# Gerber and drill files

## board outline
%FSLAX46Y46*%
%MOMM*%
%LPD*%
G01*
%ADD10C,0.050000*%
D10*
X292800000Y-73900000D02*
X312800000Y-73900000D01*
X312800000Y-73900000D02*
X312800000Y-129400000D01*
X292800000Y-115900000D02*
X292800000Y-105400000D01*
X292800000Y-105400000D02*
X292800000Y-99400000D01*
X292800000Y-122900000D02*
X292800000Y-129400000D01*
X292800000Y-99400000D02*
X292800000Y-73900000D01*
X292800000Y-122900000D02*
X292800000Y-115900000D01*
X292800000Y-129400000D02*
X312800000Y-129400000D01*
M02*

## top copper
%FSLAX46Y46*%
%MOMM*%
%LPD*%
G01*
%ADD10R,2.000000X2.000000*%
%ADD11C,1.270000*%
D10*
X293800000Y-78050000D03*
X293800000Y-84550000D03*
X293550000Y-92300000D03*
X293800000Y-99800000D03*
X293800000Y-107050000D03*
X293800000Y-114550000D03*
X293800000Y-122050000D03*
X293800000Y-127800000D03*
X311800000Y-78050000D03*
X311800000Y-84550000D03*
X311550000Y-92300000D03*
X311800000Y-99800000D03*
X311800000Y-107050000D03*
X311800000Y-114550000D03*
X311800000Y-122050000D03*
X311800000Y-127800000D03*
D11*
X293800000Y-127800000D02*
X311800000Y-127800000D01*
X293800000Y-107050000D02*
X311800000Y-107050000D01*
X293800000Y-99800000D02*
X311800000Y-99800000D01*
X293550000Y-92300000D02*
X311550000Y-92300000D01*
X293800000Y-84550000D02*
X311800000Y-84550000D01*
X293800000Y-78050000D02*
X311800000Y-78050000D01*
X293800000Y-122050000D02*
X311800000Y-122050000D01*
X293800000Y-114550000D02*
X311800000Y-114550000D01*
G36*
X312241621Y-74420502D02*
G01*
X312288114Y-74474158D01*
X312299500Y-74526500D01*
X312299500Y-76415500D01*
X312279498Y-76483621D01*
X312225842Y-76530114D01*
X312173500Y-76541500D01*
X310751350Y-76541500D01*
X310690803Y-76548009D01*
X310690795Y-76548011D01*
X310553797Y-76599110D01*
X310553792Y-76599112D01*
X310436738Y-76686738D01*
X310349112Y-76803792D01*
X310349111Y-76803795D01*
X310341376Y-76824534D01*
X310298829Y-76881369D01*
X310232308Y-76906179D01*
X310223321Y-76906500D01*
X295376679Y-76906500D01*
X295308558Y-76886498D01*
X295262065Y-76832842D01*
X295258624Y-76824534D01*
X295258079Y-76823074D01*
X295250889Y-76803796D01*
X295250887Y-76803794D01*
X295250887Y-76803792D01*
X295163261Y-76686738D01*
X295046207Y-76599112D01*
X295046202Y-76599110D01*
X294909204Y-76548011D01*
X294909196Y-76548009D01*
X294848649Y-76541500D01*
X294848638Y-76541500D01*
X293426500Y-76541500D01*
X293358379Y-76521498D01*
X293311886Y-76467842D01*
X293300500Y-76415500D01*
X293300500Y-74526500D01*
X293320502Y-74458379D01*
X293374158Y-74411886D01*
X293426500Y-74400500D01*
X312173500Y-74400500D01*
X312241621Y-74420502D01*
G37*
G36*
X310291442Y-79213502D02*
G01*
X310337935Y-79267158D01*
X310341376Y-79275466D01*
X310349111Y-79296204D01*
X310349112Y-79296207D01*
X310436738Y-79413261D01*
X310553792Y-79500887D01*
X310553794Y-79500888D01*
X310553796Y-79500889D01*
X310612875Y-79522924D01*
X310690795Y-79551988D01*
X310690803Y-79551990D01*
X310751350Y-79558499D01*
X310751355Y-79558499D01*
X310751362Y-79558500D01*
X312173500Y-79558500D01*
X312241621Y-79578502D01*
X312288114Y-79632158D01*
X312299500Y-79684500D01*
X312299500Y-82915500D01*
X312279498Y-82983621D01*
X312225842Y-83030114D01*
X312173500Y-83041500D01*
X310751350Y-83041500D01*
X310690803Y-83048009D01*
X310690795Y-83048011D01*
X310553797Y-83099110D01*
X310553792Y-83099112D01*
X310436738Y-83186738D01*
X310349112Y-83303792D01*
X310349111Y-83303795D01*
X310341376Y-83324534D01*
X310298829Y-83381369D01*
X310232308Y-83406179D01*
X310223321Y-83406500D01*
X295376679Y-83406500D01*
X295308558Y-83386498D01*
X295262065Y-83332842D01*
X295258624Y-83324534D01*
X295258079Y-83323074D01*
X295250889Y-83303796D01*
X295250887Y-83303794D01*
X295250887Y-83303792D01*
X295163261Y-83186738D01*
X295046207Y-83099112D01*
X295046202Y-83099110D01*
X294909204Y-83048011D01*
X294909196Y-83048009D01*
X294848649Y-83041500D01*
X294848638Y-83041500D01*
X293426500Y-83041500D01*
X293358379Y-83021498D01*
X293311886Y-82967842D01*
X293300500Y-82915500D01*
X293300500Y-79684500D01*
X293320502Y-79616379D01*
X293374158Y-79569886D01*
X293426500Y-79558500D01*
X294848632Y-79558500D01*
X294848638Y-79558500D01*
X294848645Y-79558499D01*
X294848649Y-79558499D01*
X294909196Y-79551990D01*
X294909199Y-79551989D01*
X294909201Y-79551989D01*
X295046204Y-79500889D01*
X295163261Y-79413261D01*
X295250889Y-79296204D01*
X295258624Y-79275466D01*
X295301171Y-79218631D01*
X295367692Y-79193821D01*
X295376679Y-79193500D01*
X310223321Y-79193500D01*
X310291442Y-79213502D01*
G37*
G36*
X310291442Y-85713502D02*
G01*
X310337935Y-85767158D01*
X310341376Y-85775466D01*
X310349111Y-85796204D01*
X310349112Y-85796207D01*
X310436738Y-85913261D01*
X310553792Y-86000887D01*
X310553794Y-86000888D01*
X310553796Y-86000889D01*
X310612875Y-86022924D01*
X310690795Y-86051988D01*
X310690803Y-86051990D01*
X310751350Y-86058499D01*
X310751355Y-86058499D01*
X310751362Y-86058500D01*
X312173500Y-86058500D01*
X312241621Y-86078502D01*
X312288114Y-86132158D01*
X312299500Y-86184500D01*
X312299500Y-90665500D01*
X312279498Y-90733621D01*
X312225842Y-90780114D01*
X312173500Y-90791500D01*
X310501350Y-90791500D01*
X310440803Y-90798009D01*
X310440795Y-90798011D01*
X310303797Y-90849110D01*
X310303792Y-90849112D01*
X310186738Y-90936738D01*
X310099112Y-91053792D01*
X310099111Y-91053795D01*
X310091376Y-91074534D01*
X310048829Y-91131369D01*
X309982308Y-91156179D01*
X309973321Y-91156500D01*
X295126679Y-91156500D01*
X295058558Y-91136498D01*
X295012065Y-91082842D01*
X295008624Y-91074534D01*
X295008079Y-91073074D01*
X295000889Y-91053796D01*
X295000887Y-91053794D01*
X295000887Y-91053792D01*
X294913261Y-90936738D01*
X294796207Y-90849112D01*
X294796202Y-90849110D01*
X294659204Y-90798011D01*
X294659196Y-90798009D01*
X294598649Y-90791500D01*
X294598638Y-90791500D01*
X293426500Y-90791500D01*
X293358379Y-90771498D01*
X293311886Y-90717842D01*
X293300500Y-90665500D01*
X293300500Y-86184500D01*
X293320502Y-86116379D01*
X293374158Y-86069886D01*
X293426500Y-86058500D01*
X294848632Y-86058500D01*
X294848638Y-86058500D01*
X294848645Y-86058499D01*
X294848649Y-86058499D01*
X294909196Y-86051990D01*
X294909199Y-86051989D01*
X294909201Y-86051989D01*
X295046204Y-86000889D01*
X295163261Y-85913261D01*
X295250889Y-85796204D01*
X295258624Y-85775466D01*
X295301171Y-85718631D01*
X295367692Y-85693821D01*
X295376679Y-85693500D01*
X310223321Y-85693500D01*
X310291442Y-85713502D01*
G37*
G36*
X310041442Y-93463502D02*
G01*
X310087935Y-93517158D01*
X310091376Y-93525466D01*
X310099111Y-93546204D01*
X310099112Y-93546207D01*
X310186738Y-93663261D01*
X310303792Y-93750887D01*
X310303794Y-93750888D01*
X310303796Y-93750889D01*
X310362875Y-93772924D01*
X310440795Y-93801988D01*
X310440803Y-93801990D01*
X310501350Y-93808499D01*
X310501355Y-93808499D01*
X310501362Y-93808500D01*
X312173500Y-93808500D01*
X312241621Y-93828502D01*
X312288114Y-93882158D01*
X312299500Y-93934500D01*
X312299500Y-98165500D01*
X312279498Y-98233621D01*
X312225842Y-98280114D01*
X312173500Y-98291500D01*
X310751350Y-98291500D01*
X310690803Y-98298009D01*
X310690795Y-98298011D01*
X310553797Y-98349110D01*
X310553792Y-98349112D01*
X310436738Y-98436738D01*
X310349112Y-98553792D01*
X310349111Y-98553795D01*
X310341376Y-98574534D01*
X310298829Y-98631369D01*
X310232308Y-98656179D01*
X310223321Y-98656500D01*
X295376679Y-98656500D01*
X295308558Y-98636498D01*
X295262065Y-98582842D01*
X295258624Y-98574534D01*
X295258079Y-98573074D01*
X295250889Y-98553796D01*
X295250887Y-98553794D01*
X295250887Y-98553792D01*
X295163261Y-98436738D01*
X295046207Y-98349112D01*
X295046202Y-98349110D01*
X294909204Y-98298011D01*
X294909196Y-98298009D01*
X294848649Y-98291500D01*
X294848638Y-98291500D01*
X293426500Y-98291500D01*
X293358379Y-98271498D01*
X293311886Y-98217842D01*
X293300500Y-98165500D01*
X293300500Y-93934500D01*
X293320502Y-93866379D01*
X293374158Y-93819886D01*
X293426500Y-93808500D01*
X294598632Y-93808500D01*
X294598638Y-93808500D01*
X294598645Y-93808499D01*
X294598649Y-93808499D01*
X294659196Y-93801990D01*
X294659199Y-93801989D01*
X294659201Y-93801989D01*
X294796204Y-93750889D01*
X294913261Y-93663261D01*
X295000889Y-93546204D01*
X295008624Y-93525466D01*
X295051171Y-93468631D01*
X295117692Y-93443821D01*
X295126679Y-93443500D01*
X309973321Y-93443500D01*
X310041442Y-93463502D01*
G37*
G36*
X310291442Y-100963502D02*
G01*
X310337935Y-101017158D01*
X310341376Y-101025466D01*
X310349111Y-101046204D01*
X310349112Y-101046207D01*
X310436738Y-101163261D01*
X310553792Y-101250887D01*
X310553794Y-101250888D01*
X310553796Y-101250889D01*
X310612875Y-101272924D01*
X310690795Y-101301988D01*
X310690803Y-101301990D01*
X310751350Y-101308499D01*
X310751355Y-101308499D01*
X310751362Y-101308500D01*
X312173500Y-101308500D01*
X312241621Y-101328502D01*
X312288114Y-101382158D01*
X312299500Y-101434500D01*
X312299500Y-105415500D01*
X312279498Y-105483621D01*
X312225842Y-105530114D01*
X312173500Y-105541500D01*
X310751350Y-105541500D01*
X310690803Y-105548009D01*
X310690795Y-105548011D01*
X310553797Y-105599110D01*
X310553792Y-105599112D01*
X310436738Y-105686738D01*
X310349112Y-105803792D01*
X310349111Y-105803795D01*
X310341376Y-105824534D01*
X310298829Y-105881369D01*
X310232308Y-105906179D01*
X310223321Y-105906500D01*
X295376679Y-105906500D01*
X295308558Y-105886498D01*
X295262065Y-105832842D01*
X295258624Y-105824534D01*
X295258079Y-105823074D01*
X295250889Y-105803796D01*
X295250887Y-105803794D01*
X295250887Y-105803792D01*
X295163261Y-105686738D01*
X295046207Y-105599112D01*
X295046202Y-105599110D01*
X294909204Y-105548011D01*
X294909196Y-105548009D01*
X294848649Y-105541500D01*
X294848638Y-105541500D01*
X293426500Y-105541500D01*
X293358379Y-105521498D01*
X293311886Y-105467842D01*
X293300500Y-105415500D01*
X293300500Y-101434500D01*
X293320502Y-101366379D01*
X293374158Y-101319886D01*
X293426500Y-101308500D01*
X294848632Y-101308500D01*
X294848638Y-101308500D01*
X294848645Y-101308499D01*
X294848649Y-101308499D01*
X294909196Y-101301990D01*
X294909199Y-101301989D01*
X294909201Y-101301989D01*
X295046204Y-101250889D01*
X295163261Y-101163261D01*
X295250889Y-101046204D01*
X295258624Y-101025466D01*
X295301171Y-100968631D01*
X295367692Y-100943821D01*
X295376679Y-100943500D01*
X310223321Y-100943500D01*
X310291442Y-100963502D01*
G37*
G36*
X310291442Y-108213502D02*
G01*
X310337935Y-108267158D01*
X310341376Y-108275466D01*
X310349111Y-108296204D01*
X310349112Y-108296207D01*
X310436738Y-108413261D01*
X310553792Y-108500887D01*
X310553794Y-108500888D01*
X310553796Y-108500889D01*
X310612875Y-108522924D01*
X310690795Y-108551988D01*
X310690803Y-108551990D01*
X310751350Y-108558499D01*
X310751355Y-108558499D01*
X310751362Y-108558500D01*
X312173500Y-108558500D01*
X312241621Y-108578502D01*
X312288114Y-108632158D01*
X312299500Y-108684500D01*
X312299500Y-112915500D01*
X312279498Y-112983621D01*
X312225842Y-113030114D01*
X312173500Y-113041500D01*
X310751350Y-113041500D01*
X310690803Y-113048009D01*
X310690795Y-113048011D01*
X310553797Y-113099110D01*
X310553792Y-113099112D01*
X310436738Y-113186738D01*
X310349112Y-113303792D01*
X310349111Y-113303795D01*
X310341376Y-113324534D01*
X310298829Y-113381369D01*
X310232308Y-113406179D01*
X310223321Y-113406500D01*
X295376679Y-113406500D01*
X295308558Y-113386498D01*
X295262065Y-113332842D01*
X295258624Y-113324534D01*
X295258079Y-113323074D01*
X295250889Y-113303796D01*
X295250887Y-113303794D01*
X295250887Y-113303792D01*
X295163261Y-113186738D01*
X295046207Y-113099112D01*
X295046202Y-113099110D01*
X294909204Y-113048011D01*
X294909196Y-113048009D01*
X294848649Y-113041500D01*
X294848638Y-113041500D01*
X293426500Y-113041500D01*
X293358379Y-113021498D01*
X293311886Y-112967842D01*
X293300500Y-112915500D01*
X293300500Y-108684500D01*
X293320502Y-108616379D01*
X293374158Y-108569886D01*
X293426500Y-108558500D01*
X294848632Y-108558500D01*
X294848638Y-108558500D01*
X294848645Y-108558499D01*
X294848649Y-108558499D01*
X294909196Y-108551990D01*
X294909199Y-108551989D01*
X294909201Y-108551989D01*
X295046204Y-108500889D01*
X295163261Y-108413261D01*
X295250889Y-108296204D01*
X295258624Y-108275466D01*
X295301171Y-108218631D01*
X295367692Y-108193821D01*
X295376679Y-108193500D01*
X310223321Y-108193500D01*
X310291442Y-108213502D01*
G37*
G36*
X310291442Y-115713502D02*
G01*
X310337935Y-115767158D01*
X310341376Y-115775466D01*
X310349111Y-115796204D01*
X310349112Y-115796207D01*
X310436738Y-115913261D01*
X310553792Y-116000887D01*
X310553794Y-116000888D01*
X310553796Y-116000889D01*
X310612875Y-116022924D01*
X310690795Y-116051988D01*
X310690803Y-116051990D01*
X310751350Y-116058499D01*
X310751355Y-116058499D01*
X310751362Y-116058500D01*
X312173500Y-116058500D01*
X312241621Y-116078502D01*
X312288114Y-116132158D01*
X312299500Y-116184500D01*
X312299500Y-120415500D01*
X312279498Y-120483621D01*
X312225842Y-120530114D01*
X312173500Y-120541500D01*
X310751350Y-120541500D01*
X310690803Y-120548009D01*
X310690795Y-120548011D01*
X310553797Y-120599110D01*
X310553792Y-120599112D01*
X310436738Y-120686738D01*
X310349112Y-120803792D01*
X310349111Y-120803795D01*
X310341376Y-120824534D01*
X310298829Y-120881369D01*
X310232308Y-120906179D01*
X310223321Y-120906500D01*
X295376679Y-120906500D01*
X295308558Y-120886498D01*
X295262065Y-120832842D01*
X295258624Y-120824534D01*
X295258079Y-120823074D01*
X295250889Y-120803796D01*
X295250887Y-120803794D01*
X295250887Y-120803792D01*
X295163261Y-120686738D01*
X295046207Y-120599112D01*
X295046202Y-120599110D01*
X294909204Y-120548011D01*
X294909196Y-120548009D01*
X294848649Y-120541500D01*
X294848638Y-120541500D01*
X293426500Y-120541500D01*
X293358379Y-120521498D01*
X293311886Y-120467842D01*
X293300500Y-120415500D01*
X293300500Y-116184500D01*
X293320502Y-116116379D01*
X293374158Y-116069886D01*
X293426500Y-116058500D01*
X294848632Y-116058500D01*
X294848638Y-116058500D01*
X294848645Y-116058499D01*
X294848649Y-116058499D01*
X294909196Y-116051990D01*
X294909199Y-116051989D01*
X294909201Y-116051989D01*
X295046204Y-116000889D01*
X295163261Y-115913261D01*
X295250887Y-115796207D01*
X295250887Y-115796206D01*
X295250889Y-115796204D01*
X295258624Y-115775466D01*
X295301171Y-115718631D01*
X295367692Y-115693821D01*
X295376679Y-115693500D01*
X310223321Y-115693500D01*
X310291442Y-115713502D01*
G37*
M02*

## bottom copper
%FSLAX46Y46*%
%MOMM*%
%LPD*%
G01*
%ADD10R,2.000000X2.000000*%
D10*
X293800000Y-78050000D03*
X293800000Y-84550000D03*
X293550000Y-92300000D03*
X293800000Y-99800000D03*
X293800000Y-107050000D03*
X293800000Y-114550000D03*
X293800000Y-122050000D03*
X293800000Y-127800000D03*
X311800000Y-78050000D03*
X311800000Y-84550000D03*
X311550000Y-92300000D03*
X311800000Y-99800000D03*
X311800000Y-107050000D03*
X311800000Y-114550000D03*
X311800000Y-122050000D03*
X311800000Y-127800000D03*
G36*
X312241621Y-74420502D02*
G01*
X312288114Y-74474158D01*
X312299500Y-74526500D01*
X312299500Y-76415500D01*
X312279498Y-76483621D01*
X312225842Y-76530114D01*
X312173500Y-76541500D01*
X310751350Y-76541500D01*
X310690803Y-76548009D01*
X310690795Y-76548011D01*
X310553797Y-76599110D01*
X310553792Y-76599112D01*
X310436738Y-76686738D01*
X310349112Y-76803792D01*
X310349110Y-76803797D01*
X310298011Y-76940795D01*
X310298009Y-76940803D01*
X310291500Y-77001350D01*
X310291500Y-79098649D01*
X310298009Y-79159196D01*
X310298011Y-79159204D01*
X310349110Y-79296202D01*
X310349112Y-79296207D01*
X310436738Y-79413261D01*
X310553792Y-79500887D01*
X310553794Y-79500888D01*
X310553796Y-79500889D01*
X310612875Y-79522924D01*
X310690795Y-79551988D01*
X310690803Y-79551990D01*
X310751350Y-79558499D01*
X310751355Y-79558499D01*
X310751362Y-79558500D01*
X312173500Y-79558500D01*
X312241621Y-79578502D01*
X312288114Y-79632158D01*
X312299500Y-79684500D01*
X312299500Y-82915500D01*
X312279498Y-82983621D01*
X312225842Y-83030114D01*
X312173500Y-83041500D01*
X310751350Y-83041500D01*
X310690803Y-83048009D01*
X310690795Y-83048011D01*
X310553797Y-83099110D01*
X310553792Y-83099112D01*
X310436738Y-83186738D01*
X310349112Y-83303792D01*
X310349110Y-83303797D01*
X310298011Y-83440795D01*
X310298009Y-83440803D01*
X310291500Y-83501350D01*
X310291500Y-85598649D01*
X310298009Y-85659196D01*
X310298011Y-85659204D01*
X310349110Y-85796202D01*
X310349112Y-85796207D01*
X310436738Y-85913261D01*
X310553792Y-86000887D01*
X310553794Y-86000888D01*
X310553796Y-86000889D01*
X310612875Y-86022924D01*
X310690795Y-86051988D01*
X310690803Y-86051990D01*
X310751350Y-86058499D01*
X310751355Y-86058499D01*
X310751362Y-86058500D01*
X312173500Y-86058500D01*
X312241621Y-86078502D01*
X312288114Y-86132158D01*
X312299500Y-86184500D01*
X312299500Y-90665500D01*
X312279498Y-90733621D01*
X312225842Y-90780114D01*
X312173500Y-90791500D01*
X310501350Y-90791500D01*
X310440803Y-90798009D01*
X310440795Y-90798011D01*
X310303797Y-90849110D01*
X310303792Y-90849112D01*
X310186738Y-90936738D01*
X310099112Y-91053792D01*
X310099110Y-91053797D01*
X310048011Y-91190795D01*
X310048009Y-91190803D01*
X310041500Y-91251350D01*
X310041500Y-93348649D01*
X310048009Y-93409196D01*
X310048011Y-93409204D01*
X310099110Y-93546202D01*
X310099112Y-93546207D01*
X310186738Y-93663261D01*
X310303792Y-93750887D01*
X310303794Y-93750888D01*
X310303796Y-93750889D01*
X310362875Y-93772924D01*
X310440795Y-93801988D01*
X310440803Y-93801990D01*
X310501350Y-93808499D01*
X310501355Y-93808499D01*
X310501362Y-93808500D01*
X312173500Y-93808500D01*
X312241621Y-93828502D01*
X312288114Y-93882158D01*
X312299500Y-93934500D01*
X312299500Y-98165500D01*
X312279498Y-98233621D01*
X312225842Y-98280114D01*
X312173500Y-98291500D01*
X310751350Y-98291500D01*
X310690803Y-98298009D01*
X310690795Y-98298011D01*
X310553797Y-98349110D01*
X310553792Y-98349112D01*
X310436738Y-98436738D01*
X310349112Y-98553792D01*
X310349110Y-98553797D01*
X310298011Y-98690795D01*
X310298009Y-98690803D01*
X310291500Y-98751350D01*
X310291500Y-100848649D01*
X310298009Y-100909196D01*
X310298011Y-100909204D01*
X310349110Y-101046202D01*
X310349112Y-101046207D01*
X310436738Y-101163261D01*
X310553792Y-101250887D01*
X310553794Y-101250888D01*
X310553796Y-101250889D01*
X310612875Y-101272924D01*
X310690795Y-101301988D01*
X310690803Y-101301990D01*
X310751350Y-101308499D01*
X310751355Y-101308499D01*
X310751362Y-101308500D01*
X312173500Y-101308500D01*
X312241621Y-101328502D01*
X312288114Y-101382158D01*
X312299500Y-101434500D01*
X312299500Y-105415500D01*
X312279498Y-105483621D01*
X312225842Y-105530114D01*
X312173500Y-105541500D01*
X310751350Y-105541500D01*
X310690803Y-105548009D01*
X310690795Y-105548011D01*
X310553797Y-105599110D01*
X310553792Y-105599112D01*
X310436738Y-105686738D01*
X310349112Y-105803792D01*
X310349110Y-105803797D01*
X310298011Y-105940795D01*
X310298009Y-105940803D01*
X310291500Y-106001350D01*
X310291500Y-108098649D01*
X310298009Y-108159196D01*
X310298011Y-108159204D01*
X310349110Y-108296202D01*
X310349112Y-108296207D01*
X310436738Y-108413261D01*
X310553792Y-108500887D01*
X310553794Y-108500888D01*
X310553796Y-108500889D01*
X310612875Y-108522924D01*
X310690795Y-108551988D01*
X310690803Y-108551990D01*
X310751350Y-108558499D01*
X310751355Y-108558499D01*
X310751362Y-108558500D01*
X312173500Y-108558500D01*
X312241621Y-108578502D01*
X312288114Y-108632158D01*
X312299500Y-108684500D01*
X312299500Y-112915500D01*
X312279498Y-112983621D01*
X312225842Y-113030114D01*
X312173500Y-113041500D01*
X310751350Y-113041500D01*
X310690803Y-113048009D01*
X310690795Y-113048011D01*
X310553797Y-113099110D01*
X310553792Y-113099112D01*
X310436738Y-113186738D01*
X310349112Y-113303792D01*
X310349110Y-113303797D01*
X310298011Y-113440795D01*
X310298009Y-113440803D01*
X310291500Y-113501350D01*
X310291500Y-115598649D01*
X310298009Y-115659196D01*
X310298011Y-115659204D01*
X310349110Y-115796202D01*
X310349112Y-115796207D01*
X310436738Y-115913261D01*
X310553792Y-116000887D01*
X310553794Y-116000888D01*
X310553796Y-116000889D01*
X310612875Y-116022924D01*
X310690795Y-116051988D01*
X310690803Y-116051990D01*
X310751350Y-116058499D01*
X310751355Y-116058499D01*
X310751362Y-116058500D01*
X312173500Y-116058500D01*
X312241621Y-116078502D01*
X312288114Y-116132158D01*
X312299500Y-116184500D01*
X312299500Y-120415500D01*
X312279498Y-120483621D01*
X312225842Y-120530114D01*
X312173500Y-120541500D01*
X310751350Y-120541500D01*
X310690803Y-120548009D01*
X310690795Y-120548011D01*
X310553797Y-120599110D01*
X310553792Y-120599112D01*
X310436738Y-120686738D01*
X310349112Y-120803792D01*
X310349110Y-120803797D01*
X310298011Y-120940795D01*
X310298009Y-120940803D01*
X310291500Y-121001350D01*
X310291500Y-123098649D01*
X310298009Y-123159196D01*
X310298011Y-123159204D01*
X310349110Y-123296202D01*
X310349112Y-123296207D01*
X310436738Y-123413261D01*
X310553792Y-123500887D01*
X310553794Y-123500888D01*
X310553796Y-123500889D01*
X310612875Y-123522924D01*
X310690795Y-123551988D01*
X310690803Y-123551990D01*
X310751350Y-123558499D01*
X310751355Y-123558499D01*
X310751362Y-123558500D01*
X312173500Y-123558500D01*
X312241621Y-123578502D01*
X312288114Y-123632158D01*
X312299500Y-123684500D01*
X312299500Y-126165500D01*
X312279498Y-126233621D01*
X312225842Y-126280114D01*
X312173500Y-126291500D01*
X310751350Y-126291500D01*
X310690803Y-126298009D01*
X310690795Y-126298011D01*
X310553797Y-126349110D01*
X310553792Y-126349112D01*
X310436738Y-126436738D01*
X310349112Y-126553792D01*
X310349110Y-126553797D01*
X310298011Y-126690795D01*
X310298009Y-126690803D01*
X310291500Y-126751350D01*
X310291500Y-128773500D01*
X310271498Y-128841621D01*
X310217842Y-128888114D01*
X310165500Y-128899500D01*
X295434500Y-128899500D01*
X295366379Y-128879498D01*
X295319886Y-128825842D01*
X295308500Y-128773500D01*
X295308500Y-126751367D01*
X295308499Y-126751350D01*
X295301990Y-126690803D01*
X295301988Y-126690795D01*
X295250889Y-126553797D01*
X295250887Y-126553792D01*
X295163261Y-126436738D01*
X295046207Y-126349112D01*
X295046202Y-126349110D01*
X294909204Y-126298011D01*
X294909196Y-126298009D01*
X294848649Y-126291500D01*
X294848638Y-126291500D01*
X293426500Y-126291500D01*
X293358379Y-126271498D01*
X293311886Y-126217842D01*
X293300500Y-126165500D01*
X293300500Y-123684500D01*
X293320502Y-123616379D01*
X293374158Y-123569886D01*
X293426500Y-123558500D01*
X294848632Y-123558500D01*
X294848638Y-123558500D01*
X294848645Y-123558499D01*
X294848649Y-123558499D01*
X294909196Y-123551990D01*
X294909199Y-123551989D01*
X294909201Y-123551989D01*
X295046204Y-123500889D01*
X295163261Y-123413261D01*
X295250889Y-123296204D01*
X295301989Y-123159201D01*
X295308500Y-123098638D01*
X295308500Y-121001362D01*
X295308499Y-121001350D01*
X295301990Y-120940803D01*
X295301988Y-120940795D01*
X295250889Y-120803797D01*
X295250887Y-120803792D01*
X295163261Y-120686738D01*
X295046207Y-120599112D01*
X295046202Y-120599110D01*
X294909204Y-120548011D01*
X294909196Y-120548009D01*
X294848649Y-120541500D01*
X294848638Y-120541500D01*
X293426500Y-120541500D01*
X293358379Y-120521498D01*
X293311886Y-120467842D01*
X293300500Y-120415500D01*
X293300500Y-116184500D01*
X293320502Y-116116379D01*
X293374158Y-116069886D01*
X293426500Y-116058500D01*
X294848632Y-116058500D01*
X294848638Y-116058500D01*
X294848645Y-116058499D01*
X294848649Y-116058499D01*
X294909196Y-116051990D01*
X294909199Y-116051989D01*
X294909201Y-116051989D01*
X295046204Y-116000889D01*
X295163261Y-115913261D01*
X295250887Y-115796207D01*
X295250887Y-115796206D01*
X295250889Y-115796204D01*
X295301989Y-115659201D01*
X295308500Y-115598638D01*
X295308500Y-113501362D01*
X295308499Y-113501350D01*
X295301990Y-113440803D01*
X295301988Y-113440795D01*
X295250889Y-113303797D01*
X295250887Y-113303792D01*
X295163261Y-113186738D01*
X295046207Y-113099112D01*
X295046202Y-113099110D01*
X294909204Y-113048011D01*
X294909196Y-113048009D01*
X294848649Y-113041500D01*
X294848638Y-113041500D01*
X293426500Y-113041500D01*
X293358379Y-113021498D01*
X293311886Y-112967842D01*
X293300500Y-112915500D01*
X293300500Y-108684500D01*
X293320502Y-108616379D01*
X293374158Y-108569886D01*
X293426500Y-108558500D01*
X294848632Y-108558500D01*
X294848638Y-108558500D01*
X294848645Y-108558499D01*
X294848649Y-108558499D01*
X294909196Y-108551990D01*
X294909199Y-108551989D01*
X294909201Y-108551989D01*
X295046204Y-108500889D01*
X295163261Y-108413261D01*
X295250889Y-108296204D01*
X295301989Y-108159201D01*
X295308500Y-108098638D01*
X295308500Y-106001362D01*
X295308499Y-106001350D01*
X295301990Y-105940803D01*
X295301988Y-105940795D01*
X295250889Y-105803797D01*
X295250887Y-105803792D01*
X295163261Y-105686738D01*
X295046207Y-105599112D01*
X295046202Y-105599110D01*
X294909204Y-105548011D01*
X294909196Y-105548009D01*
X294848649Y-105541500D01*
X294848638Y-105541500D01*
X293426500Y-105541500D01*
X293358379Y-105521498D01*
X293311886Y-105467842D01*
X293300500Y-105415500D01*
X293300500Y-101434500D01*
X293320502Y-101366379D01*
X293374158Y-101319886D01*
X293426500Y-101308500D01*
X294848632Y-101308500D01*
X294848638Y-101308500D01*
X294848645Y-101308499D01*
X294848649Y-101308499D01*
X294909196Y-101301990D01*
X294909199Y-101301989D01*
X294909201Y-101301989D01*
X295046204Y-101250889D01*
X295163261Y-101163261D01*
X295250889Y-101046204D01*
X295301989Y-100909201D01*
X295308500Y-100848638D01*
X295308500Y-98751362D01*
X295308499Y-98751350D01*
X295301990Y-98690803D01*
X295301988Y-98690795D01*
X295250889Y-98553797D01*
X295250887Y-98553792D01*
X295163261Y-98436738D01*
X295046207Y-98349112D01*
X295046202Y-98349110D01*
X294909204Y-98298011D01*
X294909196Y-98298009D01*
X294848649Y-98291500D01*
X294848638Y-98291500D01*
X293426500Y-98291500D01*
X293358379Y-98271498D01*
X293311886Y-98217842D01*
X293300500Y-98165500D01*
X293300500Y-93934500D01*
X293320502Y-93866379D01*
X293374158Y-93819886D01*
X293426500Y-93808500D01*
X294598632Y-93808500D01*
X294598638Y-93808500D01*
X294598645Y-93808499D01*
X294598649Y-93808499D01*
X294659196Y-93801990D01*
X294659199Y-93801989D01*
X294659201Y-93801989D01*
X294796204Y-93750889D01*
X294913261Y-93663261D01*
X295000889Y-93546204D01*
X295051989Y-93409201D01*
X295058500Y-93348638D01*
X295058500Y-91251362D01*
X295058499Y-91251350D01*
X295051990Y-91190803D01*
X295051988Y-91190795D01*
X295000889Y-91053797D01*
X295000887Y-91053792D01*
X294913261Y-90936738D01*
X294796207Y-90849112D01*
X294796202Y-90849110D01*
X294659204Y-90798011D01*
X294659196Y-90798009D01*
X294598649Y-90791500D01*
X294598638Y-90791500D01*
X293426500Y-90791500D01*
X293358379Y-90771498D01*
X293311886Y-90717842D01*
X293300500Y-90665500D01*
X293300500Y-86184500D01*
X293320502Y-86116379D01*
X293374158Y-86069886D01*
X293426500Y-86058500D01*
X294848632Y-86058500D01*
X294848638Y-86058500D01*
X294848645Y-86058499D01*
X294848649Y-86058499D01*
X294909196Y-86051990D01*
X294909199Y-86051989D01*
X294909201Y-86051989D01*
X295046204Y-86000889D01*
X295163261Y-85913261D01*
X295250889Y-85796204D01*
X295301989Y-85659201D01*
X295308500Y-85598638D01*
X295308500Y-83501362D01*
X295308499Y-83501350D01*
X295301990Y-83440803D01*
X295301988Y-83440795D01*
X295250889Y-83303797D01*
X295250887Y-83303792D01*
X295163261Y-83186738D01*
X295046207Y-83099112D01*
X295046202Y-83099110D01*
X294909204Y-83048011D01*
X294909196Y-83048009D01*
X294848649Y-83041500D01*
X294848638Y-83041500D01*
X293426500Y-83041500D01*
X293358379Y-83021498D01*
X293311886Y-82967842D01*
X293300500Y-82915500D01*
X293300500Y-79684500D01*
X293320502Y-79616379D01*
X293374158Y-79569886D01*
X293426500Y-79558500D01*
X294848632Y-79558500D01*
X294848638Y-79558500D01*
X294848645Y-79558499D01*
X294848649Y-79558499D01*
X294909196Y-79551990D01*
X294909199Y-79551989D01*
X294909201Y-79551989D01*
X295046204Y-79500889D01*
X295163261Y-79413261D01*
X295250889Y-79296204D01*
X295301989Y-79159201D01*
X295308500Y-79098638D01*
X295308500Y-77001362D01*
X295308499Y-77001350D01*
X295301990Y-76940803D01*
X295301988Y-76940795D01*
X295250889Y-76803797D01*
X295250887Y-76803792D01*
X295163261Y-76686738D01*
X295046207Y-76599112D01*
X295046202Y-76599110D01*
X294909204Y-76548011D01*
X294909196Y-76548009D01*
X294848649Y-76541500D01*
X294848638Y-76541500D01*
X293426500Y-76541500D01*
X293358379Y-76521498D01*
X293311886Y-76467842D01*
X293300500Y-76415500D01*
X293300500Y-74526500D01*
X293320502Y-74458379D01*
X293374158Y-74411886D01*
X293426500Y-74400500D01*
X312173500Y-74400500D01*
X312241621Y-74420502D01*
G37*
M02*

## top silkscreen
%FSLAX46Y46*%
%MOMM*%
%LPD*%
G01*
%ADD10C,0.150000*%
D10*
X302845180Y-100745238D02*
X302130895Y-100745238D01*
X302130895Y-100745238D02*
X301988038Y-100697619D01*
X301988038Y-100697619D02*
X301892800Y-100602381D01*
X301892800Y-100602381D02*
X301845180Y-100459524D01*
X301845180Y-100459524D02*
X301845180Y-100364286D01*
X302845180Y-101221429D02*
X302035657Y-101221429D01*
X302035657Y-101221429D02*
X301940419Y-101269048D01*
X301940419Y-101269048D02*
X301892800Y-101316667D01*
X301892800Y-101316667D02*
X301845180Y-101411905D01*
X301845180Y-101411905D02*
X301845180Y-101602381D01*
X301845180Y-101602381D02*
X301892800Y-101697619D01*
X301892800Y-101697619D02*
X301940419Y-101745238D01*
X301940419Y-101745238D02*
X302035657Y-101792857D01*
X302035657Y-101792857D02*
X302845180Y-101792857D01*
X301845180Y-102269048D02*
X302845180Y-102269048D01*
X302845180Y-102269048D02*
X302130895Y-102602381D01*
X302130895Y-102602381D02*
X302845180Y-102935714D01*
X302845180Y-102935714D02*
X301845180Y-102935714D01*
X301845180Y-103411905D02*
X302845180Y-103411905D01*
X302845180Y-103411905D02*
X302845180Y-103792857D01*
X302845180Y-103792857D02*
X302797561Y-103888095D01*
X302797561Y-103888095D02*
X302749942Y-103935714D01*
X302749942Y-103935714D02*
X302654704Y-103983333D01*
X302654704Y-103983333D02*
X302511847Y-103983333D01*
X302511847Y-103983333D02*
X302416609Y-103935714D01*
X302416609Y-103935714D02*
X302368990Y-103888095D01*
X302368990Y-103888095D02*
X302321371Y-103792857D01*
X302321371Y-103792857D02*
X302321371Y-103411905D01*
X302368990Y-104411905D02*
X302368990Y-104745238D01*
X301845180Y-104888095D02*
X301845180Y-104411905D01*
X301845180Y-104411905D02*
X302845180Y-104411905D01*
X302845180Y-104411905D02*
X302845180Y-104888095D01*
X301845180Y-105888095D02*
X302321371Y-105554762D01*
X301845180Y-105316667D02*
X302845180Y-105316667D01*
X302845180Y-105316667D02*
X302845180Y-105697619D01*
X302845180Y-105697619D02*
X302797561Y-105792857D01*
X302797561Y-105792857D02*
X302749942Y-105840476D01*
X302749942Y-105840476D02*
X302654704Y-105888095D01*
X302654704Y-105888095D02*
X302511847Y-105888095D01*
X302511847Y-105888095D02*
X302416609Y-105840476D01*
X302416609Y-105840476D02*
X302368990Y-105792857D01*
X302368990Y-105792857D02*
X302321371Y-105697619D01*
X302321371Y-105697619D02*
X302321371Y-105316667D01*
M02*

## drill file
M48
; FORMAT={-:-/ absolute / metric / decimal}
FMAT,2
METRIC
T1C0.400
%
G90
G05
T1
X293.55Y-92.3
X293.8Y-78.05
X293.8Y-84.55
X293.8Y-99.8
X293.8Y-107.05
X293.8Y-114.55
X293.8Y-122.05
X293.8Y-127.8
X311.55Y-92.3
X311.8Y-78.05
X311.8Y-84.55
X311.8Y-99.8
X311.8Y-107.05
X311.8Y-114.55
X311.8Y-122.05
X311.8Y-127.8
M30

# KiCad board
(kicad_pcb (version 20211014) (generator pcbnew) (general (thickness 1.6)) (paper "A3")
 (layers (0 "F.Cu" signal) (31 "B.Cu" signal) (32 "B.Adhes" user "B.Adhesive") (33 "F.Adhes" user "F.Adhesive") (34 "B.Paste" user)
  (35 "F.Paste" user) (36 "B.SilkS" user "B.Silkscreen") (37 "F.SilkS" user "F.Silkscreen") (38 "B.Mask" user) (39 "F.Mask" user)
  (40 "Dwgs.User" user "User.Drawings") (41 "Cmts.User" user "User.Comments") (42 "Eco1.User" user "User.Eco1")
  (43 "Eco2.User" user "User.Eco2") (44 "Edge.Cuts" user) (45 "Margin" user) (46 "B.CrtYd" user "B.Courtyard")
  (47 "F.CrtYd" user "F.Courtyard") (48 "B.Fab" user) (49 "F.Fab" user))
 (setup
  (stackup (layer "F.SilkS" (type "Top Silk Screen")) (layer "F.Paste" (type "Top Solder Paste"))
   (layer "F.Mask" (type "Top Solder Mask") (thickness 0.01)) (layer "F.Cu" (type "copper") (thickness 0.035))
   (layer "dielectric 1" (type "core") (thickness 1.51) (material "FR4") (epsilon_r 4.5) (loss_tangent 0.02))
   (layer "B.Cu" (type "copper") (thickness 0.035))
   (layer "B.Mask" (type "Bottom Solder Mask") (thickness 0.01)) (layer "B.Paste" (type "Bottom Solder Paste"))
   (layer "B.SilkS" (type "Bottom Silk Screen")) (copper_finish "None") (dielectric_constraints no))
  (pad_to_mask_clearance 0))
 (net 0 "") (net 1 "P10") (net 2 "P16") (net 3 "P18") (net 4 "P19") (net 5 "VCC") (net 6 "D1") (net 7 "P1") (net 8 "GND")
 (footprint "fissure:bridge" (layer "F.Cu") (at 293.8 107.55 90)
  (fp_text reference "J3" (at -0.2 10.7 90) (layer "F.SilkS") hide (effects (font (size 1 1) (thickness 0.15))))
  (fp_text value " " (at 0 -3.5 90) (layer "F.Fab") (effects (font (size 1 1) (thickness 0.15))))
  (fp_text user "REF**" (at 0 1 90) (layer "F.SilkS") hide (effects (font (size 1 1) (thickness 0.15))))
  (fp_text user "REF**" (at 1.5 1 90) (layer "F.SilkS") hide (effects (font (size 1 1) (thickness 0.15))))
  (pad "1" thru_hole rect (at 29.5 0 90) (size 2 2) (drill 0.4) (layers *.Cu *.Mask) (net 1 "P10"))
  (pad "2" thru_hole rect (at 23 0 90) (size 2 2) (drill 0.4) (layers F&B.Cu *.Mask) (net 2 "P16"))
  (pad "3" thru_hole rect (at 15.25 -0.25 90) (size 2 2) (drill 0.4) (layers F&B.Cu *.Mask) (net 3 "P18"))
  (pad "4" thru_hole rect (at 7.75 0 90) (size 2 2) (drill 0.4) (layers F&B.Cu *.Mask) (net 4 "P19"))
  (pad "5" thru_hole rect (at 0.5 0 90) (size 2 2) (drill 0.4) (layers F&B.Cu *.Mask) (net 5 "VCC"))
  (pad "6" thru_hole rect (at -7 0 90) (size 2 2) (drill 0.4) (layers F&B.Cu *.Mask) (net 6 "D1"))
  (pad "7" thru_hole rect (at -14.5 0 90) (size 2 2) (drill 0.4) (layers F&B.Cu *.Mask) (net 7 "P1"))
  (pad "8" thru_hole rect (at -20.25 0 90) (size 2 2) (drill 0.4) (layers F&B.Cu *.Mask) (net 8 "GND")))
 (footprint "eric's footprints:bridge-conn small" (layer "F.Cu") (at 311.8 107.55 90)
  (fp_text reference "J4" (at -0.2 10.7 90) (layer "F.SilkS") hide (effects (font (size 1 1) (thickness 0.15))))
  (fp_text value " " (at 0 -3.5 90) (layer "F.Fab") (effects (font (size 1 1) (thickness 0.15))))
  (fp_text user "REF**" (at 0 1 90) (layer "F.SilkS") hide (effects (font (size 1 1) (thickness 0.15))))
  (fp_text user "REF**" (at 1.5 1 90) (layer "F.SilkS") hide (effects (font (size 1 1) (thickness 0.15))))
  (pad "1" thru_hole rect (at 29.5 0 90) (size 2 2) (drill 0.4) (layers F&B.Cu *.Mask) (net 1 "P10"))
  (pad "2" thru_hole rect (at 23 0 90) (size 2 2) (drill 0.4) (layers F&B.Cu *.Mask) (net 2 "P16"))
  (pad "3" thru_hole rect (at 15.25 -0.25 90) (size 2 2) (drill 0.4) (layers F&B.Cu *.Mask) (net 3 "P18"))
  (pad "4" thru_hole rect (at 7.75 0 90) (size 2 2) (drill 0.4) (layers F&B.Cu *.Mask) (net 4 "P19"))
  (pad "5" thru_hole rect (at 0.5 0 90) (size 2 2) (drill 0.4) (layers F&B.Cu *.Mask) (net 5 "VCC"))
  (pad "6" thru_hole rect (at -7 0 90) (size 2 2) (drill 0.4) (layers F&B.Cu *.Mask) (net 6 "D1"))
  (pad "7" thru_hole rect (at -14.5 0 90) (size 2 2) (drill 0.4) (layers F&B.Cu *.Mask) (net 7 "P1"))
  (pad "8" thru_hole rect (at -20.25 0 90) (size 2 2) (drill 0.4) (layers F&B.Cu *.Mask) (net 8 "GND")))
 (gr_line (start 292.8 73.9) (end 312.8 73.9) (layer "Edge.Cuts") (width 0.05))
 (gr_line (start 312.8 73.9) (end 312.8 129.4) (layer "Edge.Cuts") (width 0.05))
 (gr_line (start 292.8 115.9) (end 292.8 105.4) (layer "Edge.Cuts") (width 0.05))
 (gr_line (start 292.8 105.4) (end 292.8 99.4) (layer "Edge.Cuts") (width 0.05))
 (gr_line (start 292.8 122.9) (end 292.8 129.4) (layer "Edge.Cuts") (width 0.05))
 (gr_line (start 292.8 99.4) (end 292.8 73.9) (layer "Edge.Cuts") (width 0.05))
 (gr_line (start 292.8 122.9) (end 292.8 115.9) (layer "Edge.Cuts") (width 0.05))
 (gr_line (start 292.8 129.4) (end 312.8 129.4) (layer "Edge.Cuts") (width 0.05))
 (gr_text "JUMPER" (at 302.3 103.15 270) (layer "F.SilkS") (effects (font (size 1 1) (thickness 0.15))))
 (segment (start 293.8 127.8) (end 311.8 127.8) (width 1.27) (layer "F.Cu") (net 8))
 (segment (start 293.8 107.05) (end 311.8 107.05) (width 1.27) (layer "F.Cu") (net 5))
 (segment (start 293.8 99.8) (end 311.8 99.8) (width 1.27) (layer "F.Cu") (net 4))
 (segment (start 293.55 92.3) (end 311.55 92.3) (width 1.27) (layer "F.Cu") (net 3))
 (segment (start 293.8 84.55) (end 311.8 84.55) (width 1.27) (layer "F.Cu") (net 2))
 (segment (start 293.8 78.05) (end 311.8 78.05) (width 1.27) (layer "F.Cu") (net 1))
 (segment (start 293.8 122.05) (end 311.8 122.05) (width 1.27) (layer "F.Cu") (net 7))
 (segment (start 293.8 114.55) (end 311.8 114.55) (width 1.27) (layer "F.Cu") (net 6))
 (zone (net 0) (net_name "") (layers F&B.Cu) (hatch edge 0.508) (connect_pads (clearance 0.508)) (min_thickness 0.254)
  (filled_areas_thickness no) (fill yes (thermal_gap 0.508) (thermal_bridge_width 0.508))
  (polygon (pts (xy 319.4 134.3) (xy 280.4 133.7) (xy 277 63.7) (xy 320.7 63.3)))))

